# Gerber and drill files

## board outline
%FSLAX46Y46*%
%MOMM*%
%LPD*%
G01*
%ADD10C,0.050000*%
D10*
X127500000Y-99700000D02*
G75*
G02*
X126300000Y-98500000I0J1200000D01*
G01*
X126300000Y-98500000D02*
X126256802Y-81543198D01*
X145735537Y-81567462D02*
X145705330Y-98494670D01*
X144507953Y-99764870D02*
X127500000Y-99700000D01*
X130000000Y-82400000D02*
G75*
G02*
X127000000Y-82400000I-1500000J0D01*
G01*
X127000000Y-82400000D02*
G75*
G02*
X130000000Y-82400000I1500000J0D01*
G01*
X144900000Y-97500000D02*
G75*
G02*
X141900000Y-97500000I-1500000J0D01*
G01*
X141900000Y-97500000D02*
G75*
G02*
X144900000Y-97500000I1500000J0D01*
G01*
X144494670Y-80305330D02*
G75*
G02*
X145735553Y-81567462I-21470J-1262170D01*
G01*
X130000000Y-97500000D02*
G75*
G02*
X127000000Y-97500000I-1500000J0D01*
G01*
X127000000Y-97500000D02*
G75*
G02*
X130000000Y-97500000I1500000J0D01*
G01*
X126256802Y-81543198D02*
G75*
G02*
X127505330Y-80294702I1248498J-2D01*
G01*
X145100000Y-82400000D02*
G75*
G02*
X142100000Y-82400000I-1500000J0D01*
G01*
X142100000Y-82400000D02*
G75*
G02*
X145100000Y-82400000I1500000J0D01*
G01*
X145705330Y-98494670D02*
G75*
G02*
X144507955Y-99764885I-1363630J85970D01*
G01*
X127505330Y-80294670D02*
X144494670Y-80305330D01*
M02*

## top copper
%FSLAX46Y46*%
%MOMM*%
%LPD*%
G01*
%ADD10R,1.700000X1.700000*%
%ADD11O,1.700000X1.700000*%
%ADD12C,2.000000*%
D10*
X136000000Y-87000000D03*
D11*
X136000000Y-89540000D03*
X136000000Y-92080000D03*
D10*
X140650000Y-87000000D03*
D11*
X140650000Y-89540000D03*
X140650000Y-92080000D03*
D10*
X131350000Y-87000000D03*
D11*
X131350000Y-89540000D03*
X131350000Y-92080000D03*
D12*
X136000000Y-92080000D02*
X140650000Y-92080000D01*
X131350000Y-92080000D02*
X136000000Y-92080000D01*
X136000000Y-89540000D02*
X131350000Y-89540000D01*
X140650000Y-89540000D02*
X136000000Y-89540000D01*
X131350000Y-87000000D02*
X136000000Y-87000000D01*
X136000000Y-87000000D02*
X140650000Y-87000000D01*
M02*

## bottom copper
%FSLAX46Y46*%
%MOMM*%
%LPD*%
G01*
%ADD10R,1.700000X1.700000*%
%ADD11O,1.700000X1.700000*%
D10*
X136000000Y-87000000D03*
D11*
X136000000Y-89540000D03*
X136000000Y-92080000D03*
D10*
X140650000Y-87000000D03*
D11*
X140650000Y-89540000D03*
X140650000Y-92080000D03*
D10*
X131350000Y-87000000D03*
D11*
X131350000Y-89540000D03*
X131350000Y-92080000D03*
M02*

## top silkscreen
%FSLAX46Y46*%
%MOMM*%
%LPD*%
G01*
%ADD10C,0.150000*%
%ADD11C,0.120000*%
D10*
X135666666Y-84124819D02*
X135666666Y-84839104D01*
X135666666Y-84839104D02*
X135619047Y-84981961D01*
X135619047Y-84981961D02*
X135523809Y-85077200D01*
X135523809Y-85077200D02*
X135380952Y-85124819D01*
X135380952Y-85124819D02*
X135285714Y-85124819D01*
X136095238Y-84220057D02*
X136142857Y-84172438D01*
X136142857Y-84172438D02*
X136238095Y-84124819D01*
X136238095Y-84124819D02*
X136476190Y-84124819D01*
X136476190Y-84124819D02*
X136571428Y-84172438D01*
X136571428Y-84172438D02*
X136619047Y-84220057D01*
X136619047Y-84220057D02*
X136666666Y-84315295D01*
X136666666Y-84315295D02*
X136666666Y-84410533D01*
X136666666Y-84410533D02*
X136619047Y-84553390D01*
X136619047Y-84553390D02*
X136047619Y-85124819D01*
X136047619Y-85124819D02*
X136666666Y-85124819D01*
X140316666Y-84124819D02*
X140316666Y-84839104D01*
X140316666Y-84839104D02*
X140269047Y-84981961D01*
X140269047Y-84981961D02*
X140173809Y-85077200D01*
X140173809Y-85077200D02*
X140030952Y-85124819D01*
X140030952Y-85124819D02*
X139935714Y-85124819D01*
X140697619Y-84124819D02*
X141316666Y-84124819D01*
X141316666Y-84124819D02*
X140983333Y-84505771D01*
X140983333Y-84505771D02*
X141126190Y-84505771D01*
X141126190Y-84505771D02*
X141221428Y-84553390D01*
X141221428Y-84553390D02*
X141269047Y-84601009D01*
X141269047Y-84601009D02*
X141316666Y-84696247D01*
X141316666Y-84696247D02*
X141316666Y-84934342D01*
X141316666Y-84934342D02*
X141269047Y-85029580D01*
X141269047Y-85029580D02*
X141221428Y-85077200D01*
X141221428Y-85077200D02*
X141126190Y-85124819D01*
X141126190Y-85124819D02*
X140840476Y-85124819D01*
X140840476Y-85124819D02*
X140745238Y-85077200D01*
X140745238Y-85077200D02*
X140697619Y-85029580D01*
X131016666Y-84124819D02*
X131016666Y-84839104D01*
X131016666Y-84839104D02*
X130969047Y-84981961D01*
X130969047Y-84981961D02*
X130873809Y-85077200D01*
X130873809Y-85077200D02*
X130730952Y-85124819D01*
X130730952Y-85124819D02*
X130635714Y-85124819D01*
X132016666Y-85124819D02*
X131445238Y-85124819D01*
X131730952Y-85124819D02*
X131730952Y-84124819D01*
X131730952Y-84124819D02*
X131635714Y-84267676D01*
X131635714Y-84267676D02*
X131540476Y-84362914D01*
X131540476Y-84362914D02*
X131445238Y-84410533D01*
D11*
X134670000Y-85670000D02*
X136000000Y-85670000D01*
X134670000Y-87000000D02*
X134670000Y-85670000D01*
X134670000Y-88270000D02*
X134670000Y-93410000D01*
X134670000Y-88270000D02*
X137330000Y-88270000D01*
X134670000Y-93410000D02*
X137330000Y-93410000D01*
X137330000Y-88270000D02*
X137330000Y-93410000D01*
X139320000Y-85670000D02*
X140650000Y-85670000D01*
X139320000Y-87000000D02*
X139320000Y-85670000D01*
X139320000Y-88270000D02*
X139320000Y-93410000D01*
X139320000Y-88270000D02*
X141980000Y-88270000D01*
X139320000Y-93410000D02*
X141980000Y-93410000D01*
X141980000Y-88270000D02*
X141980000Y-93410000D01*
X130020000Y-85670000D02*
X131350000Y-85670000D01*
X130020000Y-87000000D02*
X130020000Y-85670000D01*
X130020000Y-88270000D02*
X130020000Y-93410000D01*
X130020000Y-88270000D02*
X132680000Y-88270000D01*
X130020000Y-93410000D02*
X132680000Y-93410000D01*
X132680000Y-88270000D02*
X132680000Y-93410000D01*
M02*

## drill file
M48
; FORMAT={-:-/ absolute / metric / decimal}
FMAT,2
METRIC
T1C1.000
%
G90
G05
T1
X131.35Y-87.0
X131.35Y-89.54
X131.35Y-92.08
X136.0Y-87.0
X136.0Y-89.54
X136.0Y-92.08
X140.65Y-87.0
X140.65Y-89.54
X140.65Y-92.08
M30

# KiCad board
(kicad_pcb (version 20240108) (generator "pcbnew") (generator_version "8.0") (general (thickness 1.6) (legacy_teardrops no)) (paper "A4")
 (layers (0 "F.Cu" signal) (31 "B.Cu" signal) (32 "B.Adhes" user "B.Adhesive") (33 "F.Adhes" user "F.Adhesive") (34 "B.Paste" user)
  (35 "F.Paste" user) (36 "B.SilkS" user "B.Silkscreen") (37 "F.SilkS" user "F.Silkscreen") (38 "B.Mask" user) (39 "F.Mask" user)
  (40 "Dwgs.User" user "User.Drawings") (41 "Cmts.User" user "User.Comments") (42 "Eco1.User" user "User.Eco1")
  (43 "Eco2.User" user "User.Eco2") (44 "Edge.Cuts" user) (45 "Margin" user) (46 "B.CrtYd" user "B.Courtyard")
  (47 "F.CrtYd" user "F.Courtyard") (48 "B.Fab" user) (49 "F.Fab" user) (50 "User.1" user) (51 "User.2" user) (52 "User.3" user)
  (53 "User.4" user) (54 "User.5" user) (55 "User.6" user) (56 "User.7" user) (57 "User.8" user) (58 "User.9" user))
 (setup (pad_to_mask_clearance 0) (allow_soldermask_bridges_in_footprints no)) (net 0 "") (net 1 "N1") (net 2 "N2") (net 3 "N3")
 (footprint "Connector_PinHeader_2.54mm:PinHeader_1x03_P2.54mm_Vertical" (layer "F.Cu") (at 136 87)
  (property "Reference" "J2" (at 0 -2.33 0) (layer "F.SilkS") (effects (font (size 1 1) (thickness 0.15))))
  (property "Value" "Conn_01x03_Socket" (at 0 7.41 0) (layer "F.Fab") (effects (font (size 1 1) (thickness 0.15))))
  (fp_line (start -1.33 -1.33) (end 0 -1.33) (stroke (width 0.12) (type solid)) (layer "F.SilkS"))
  (fp_line (start -1.33 0) (end -1.33 -1.33) (stroke (width 0.12) (type solid)) (layer "F.SilkS"))
  (fp_line (start -1.33 1.27) (end -1.33 6.41) (stroke (width 0.12) (type solid)) (layer "F.SilkS"))
  (fp_line (start -1.33 1.27) (end 1.33 1.27) (stroke (width 0.12) (type solid)) (layer "F.SilkS"))
  (fp_line (start -1.33 6.41) (end 1.33 6.41) (stroke (width 0.12) (type solid)) (layer "F.SilkS"))
  (fp_line (start 1.33 1.27) (end 1.33 6.41) (stroke (width 0.12) (type solid)) (layer "F.SilkS"))
  (pad "1" thru_hole rect (at 0 0) (size 1.7 1.7) (drill 1) (layers "*.Cu" "*.Mask") (remove_unused_layers no) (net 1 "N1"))
  (pad "2" thru_hole oval (at 0 2.54) (size 1.7 1.7) (drill 1) (layers "*.Cu" "*.Mask") (remove_unused_layers no) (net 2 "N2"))
  (pad "3" thru_hole oval (at 0 5.08) (size 1.7 1.7) (drill 1) (layers "*.Cu" "*.Mask") (remove_unused_layers no) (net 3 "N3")))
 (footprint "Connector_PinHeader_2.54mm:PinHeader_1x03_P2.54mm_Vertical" (layer "F.Cu") (at 140.65 87)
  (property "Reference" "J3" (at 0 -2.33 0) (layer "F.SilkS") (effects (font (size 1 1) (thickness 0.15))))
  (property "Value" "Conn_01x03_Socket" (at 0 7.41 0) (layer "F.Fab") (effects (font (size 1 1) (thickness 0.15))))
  (fp_line (start -1.33 -1.33) (end 0 -1.33) (stroke (width 0.12) (type solid)) (layer "F.SilkS"))
  (fp_line (start -1.33 0) (end -1.33 -1.33) (stroke (width 0.12) (type solid)) (layer "F.SilkS"))
  (fp_line (start -1.33 1.27) (end -1.33 6.41) (stroke (width 0.12) (type solid)) (layer "F.SilkS"))
  (fp_line (start -1.33 1.27) (end 1.33 1.27) (stroke (width 0.12) (type solid)) (layer "F.SilkS"))
  (fp_line (start -1.33 6.41) (end 1.33 6.41) (stroke (width 0.12) (type solid)) (layer "F.SilkS"))
  (fp_line (start 1.33 1.27) (end 1.33 6.41) (stroke (width 0.12) (type solid)) (layer "F.SilkS"))
  (pad "1" thru_hole rect (at 0 0) (size 1.7 1.7) (drill 1) (layers "*.Cu" "*.Mask") (remove_unused_layers no) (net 1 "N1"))
  (pad "2" thru_hole oval (at 0 2.54) (size 1.7 1.7) (drill 1) (layers "*.Cu" "*.Mask") (remove_unused_layers no) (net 2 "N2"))
  (pad "3" thru_hole oval (at 0 5.08) (size 1.7 1.7) (drill 1) (layers "*.Cu" "*.Mask") (remove_unused_layers no) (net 3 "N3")))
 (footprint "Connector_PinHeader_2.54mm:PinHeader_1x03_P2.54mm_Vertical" (layer "F.Cu") (at 131.35 87)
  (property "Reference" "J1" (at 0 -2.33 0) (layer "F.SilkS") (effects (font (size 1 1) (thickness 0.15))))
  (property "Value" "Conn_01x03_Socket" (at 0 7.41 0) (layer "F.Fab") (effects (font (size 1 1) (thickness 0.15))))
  (fp_line (start -1.33 -1.33) (end 0 -1.33) (stroke (width 0.12) (type solid)) (layer "F.SilkS"))
  (fp_line (start -1.33 0) (end -1.33 -1.33) (stroke (width 0.12) (type solid)) (layer "F.SilkS"))
  (fp_line (start -1.33 1.27) (end -1.33 6.41) (stroke (width 0.12) (type solid)) (layer "F.SilkS"))
  (fp_line (start -1.33 1.27) (end 1.33 1.27) (stroke (width 0.12) (type solid)) (layer "F.SilkS"))
  (fp_line (start -1.33 6.41) (end 1.33 6.41) (stroke (width 0.12) (type solid)) (layer "F.SilkS"))
  (fp_line (start 1.33 1.27) (end 1.33 6.41) (stroke (width 0.12) (type solid)) (layer "F.SilkS"))
  (pad "1" thru_hole rect (at 0 0) (size 1.7 1.7) (drill 1) (layers "*.Cu" "*.Mask") (remove_unused_layers no) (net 1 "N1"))
  (pad "2" thru_hole oval (at 0 2.54) (size 1.7 1.7) (drill 1) (layers "*.Cu" "*.Mask") (remove_unused_layers no) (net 2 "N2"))
  (pad "3" thru_hole oval (at 0 5.08) (size 1.7 1.7) (drill 1) (layers "*.Cu" "*.Mask") (remove_unused_layers no) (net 3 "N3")))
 (gr_arc (start 127.5 99.7) (mid 126.651472 99.348528) (end 126.3 98.5) (stroke (width 0.05) (type default)) (layer "Edge.Cuts"))
 (gr_line (start 126.3 98.5) (end 126.256802 81.543198) (stroke (width 0.05) (type default)) (layer "Edge.Cuts"))
 (gr_line (start 145.735537 81.567462) (end 145.70533 98.49467) (stroke (width 0.05) (type default)) (layer "Edge.Cuts"))
 (gr_line (start 144.507953 99.76487) (end 127.5 99.7) (stroke (width 0.05) (type default)) (layer "Edge.Cuts"))
 (gr_circle (center 128.5 82.4) (end 130 82.4) (stroke (width 0.05) (type default)) (fill none) (layer "Edge.Cuts"))
 (gr_circle (center 143.4 97.5) (end 144.9 97.5) (stroke (width 0.05) (type default)) (fill none) (layer "Edge.Cuts"))
 (gr_arc (start 144.49467 80.30533) (mid 145.373365 80.682486) (end 145.735537 81.567462) (stroke (width 0.05) (type default))
  (layer "Edge.Cuts"))
 (gr_circle (center 128.5 97.5) (end 130 97.5) (stroke (width 0.05) (type default)) (fill none) (layer "Edge.Cuts"))
 (gr_arc (start 126.256802 81.543198) (mid 126.622487 80.660355) (end 127.50533 80.29467) (stroke (width 0.05) (type default))
  (layer "Edge.Cuts"))
 (gr_circle (center 143.6 82.4) (end 145.1 82.4) (stroke (width 0.05) (type default)) (fill none) (layer "Edge.Cuts"))
 (gr_arc (start 145.70533 98.49467) (mid 145.335923 99.345906) (end 144.507953 99.76487) (stroke (width 0.05) (type default))
  (layer "Edge.Cuts"))
 (gr_line (start 127.50533 80.29467) (end 144.49467 80.30533) (stroke (width 0.05) (type default)) (layer "Edge.Cuts"))
 (segment (start 136 92.08) (end 140.65 92.08) (width 2) (layer "F.Cu") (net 3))
 (segment (start 131.35 92.08) (end 136 92.08) (width 2) (layer "F.Cu") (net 3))
 (segment (start 136 89.54) (end 131.35 89.54) (width 2) (layer "F.Cu") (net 2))
 (segment (start 140.65 89.54) (end 136 89.54) (width 2) (layer "F.Cu") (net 2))
 (segment (start 131.35 87) (end 136 87) (width 2) (layer "F.Cu") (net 1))
 (segment (start 136 87) (end 140.65 87) (width 2) (layer "F.Cu") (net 1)))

